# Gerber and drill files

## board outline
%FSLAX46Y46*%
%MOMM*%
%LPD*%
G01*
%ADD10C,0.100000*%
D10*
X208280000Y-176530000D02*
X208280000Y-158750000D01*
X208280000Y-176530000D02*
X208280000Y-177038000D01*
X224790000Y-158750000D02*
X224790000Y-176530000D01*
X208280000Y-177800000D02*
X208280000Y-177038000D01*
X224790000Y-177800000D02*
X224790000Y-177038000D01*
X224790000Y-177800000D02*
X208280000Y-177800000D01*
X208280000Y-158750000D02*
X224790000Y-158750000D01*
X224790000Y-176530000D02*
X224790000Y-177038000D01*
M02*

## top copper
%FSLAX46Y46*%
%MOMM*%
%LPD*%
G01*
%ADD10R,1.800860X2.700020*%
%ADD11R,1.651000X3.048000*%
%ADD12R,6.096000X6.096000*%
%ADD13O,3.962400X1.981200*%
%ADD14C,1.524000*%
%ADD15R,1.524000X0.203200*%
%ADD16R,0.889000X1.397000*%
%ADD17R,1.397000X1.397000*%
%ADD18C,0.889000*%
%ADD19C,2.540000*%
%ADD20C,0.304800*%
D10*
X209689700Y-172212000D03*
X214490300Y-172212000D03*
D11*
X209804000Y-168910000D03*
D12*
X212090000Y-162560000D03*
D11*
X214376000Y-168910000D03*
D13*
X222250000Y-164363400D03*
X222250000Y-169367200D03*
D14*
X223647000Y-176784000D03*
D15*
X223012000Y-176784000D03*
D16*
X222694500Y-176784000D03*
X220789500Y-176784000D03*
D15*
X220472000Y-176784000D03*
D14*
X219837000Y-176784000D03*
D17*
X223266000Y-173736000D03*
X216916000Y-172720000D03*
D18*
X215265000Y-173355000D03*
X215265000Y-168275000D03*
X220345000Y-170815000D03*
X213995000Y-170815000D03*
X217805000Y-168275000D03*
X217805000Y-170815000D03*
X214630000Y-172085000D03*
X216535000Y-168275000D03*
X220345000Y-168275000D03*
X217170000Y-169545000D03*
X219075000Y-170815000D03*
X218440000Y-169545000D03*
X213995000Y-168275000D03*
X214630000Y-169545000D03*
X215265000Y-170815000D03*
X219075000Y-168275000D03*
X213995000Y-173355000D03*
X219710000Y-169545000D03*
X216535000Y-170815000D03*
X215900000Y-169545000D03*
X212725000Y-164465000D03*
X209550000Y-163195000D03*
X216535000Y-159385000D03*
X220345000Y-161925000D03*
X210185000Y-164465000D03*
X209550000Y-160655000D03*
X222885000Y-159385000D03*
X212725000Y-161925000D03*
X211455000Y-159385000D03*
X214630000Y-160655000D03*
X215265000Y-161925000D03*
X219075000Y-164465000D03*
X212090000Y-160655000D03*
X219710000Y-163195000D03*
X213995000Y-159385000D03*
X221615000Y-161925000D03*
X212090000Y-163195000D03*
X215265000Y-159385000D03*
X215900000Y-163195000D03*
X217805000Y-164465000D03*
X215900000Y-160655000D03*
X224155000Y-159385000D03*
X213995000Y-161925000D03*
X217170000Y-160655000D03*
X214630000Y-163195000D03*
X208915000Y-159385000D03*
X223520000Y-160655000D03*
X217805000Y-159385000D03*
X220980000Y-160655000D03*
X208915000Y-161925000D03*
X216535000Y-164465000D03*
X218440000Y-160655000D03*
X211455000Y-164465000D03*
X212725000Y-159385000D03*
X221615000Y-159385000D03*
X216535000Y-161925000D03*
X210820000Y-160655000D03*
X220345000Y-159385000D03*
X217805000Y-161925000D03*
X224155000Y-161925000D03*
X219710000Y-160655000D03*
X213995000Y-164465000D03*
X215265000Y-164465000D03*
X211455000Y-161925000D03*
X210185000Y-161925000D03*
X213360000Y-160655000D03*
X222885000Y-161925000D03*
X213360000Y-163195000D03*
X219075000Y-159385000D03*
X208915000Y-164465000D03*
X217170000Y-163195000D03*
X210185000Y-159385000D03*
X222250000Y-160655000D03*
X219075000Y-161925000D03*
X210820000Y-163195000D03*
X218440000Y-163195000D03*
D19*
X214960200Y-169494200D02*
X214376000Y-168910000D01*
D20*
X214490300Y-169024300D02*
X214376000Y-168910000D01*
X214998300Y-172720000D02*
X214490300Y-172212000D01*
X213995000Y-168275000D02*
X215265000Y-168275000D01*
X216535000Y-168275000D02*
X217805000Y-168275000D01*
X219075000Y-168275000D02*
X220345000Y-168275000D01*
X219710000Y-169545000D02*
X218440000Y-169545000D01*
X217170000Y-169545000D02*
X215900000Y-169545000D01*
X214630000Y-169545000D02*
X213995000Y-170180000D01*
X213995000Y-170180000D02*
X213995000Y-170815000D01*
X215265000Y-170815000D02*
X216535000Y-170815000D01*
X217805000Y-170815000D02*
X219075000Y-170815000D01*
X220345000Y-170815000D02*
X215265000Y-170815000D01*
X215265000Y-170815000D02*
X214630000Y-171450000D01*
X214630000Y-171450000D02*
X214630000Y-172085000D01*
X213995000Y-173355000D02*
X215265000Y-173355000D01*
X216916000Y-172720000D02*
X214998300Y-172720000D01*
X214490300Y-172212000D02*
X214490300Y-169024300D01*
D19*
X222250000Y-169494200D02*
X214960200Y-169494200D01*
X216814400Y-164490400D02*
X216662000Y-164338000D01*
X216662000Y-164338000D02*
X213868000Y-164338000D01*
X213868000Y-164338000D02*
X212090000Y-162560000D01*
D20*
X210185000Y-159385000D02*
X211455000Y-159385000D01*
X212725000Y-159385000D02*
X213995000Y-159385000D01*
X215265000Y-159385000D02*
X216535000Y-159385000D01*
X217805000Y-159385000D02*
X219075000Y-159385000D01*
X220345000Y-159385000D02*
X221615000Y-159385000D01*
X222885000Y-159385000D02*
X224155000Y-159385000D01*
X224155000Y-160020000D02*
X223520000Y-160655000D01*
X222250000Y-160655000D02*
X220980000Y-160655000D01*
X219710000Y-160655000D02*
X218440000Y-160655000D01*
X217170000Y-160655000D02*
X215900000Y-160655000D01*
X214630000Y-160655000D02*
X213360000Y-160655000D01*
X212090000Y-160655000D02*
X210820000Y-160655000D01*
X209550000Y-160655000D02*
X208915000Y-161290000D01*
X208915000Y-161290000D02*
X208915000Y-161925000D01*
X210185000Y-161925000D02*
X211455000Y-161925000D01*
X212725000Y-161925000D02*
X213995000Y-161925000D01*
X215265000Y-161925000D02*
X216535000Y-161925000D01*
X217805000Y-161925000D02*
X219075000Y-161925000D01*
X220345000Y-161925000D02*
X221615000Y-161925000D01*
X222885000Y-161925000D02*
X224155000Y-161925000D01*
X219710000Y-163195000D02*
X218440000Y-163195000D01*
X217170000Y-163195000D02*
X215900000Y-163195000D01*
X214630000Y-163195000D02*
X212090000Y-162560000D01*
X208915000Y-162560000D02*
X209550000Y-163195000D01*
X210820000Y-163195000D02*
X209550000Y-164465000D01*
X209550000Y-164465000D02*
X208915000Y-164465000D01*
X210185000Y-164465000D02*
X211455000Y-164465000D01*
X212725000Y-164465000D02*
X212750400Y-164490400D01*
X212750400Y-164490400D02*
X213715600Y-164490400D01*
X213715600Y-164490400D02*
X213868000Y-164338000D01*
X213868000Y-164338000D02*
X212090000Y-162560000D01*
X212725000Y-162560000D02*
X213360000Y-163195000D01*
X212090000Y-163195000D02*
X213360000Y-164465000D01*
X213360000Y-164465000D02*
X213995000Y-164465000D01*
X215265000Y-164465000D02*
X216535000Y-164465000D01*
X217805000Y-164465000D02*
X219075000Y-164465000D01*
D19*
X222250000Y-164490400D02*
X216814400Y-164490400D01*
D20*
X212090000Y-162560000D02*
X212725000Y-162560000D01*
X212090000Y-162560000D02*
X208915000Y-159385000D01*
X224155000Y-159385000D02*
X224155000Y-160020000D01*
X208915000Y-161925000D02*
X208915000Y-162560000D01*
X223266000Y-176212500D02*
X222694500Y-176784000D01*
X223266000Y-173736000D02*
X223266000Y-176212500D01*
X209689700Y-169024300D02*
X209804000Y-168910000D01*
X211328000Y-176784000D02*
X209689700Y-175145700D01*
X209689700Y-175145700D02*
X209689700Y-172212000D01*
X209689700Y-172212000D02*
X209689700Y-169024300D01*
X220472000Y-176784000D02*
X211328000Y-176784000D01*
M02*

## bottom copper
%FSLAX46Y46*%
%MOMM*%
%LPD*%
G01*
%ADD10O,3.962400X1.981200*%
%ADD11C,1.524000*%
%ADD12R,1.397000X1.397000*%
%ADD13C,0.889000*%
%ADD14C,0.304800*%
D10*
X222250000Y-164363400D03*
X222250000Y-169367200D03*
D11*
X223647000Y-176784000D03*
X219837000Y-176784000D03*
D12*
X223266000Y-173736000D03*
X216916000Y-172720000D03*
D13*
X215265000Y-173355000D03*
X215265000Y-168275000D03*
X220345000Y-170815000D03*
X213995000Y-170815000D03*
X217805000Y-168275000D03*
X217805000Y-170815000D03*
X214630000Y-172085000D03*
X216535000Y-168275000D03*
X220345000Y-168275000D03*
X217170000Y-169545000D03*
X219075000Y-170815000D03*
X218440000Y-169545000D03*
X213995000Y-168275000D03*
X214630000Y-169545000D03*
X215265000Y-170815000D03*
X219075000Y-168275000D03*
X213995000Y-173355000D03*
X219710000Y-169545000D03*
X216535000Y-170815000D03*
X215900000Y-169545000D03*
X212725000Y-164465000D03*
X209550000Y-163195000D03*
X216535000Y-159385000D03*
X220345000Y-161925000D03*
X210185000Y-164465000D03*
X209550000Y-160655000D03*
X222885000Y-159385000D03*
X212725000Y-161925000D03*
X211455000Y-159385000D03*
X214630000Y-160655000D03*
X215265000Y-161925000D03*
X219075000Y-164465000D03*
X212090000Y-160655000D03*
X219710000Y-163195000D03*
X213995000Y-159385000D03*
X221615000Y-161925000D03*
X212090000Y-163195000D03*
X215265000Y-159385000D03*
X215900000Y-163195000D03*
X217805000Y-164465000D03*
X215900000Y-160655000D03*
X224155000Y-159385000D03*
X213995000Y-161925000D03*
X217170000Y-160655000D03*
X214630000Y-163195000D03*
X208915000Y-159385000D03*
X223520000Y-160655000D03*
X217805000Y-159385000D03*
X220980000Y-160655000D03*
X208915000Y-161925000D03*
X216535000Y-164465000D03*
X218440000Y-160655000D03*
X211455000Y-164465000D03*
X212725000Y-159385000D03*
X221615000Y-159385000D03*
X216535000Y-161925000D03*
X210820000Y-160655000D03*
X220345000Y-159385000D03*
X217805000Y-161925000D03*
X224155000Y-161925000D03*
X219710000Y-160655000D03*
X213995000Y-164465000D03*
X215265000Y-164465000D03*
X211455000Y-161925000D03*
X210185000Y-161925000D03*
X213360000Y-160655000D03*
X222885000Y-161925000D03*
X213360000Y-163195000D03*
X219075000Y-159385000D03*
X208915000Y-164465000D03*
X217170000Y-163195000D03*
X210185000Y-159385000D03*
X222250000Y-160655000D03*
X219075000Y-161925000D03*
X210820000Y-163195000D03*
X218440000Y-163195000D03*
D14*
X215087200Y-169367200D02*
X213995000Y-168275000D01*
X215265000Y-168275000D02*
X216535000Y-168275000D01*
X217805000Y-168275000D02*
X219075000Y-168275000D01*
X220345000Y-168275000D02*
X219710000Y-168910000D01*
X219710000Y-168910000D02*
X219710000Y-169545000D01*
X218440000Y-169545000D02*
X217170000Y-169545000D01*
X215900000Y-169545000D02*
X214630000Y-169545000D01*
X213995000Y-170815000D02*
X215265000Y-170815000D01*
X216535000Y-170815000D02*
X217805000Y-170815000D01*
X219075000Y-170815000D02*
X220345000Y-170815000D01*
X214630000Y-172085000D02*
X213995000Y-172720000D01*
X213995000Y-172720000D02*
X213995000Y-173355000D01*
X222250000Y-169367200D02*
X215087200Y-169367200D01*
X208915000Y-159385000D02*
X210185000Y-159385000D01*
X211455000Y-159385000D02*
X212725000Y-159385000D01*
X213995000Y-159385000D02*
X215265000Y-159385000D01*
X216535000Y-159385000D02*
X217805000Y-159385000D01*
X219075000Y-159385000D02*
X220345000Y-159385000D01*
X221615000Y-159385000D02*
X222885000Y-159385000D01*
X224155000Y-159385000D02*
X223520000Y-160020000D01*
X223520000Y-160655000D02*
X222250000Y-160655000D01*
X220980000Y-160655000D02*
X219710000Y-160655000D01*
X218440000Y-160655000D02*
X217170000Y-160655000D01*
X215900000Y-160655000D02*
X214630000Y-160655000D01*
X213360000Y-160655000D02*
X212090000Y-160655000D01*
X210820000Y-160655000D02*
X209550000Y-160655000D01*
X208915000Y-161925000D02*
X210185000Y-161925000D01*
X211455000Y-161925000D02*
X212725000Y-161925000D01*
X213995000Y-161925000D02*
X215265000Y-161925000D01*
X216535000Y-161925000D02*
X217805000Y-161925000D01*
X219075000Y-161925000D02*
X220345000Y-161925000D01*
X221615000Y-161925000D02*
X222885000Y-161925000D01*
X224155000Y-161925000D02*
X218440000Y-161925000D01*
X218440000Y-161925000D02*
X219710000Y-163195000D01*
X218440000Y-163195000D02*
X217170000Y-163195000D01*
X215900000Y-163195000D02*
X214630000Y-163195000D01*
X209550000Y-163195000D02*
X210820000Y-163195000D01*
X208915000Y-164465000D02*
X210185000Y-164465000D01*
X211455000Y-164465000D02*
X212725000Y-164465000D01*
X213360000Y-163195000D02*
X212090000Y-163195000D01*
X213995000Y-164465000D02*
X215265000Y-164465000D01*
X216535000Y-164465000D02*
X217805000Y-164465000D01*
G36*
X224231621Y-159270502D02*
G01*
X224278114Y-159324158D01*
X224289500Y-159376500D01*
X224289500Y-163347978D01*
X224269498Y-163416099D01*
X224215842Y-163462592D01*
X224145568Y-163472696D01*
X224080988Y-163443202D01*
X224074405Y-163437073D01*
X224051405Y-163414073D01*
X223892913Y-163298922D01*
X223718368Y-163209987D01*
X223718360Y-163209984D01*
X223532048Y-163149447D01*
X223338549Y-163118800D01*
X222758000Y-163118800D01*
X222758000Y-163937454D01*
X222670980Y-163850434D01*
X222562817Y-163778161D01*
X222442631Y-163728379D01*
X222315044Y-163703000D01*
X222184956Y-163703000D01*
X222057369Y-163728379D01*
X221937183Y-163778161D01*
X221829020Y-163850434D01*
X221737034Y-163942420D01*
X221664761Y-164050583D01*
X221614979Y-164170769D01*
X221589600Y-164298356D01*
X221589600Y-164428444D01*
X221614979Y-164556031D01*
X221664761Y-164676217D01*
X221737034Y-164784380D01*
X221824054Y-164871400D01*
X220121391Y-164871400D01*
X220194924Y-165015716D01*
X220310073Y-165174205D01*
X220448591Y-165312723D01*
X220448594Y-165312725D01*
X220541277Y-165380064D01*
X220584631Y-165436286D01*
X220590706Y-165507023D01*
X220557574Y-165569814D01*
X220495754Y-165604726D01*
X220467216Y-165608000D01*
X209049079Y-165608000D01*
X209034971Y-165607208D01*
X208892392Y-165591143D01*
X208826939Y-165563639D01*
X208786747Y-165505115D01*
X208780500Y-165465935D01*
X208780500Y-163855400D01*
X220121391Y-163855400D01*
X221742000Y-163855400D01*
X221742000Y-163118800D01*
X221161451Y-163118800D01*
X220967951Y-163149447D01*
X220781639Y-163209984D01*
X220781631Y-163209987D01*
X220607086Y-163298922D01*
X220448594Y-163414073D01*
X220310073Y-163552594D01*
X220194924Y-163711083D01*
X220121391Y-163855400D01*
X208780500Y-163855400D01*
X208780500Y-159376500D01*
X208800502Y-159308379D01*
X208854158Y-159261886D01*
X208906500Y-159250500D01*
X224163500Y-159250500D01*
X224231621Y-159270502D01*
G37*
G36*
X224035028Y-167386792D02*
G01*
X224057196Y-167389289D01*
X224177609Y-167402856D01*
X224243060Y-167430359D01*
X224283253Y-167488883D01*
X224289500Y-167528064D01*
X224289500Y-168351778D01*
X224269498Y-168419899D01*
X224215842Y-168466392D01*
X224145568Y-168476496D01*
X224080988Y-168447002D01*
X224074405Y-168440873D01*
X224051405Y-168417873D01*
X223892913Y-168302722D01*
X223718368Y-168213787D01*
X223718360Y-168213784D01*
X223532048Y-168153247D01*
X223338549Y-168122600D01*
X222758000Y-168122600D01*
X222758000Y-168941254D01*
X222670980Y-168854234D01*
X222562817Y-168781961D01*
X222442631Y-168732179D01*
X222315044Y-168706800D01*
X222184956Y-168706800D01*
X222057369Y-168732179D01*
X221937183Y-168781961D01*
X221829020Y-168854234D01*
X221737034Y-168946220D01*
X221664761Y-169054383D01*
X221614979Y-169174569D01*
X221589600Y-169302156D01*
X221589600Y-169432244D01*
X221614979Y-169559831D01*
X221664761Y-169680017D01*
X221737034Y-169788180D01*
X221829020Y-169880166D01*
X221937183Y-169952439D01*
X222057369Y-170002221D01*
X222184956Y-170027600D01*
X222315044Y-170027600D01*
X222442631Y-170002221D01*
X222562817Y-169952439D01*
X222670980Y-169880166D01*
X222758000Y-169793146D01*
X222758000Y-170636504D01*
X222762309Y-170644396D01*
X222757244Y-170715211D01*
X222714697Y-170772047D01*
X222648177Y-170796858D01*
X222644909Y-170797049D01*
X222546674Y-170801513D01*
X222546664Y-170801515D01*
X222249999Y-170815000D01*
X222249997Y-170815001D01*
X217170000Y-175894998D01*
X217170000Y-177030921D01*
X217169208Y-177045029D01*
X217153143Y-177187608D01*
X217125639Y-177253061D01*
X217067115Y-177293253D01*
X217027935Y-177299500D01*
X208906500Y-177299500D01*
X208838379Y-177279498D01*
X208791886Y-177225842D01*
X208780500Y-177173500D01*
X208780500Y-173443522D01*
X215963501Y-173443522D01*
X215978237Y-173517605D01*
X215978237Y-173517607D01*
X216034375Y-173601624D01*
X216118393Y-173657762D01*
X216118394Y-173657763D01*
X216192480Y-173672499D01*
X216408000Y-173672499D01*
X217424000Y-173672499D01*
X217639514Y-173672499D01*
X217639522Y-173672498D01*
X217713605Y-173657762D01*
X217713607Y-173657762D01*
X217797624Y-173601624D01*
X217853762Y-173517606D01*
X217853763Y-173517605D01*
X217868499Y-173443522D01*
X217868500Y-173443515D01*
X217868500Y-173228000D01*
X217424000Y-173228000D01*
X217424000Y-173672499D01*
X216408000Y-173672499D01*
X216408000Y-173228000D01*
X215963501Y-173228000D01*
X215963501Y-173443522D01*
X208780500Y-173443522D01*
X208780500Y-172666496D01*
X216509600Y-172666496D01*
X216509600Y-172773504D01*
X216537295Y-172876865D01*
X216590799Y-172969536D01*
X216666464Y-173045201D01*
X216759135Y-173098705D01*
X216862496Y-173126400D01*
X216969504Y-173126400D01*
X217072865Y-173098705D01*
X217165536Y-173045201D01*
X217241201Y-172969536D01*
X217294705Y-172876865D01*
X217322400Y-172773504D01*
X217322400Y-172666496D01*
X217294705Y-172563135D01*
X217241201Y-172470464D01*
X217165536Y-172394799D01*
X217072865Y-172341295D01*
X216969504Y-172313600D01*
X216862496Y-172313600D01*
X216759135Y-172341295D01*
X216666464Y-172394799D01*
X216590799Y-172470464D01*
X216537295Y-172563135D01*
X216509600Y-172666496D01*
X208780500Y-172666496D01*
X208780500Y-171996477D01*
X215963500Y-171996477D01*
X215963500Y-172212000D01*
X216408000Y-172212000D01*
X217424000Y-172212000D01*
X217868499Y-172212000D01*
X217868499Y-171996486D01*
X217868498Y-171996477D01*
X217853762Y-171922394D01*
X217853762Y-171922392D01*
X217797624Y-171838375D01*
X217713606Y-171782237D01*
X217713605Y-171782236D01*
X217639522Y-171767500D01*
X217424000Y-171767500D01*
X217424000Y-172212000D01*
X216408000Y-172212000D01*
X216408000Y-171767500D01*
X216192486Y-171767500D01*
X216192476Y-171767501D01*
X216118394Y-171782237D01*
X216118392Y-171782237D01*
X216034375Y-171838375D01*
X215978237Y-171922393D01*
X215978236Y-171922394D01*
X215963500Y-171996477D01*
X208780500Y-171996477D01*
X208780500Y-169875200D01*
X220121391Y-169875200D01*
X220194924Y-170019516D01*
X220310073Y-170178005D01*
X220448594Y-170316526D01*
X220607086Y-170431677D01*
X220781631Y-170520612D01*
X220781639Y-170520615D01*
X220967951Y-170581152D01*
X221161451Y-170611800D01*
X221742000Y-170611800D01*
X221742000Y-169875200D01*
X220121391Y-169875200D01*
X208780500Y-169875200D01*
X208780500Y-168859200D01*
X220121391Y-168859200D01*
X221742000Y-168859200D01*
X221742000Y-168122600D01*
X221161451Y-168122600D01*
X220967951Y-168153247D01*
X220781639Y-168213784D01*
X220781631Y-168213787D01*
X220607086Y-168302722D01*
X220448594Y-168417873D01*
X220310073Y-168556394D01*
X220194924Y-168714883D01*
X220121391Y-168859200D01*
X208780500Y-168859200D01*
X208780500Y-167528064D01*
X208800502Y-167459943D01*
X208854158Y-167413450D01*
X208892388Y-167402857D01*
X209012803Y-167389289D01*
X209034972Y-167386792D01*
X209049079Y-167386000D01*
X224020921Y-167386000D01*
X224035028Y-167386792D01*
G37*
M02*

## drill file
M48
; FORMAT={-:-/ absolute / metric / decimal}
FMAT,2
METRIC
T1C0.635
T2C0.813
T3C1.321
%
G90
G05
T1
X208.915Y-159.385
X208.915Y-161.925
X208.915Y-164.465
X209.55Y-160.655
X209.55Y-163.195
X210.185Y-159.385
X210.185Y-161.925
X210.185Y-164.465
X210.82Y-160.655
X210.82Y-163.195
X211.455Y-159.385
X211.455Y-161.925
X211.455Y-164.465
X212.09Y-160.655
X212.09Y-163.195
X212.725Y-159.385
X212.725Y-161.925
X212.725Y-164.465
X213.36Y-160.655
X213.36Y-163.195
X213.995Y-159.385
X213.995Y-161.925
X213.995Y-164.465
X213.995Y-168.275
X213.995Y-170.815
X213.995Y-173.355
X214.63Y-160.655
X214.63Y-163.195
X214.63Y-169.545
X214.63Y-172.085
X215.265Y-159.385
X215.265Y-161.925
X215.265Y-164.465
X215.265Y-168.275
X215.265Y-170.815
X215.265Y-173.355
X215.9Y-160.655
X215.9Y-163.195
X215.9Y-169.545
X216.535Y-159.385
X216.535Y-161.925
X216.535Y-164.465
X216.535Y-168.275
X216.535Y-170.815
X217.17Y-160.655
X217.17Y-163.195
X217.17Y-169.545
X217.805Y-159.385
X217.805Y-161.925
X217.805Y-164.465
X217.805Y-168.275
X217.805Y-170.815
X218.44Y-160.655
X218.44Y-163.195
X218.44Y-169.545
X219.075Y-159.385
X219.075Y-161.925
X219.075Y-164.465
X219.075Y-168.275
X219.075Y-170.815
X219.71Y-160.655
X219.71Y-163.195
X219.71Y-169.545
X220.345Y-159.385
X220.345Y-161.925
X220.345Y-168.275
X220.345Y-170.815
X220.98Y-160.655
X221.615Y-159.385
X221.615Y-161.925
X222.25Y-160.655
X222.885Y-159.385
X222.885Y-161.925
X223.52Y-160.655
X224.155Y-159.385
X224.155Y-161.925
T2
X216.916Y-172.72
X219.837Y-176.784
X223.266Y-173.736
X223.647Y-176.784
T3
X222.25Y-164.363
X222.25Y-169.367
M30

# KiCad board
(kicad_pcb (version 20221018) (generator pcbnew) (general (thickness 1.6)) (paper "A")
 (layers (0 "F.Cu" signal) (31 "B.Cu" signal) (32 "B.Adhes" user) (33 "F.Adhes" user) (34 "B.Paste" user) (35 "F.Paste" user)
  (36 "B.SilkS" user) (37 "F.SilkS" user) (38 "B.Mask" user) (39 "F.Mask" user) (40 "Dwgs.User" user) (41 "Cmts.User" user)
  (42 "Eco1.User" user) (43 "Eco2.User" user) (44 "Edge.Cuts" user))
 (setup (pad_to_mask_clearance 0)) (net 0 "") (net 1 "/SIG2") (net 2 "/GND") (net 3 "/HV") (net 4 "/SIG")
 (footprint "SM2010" (layer "F.Cu") (at 212.09 172.212)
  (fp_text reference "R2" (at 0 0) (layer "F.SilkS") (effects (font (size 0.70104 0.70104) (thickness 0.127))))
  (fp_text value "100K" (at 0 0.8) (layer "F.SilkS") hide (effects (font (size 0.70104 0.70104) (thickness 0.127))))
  (pad "1" smd rect (at -2.4003 0) (size 1.80086 2.70002) (layers "F.Cu" "F.Paste" "F.Mask") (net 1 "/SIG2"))
  (pad "2" smd rect (at 2.4003 0) (size 1.80086 2.70002) (layers "F.Cu" "F.Paste" "F.Mask") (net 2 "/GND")))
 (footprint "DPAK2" (layer "F.Cu") (at 212.09 168.91)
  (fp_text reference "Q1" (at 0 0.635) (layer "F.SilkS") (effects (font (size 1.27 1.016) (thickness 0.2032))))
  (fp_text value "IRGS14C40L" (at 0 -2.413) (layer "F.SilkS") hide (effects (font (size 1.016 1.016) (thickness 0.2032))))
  (pad "1" smd rect (at -2.286 0) (size 1.651 3.048) (layers "F.Cu" "F.Paste" "F.Mask") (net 1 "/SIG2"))
  (pad "2" smd rect (at 0 -6.35) (size 6.096 6.096) (layers "F.Cu" "F.Paste" "F.Mask") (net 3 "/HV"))
  (pad "3" smd rect (at 2.286 0) (size 1.651 3.048) (layers "F.Cu" "F.Paste" "F.Mask") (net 2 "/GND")))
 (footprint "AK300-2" (layer "F.Cu") (at 222.25 166.878 -90)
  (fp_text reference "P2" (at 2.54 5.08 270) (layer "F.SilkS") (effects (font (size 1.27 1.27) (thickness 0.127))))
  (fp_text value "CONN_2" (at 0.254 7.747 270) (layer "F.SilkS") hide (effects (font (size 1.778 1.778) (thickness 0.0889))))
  (pad "1" thru_hole oval (at -2.5146 0 270) (size 1.9812 3.9624) (drill 1.3208) (layers "*.Cu" "F.Paste" "F.SilkS" "F.Mask") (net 3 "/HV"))
  (pad "2" thru_hole oval (at 2.4892 0 270) (size 1.9812 3.9624) (drill 1.3208) (layers "*.Cu" "F.Paste" "F.SilkS" "F.Mask") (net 2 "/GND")))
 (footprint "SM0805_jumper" (layer "F.Cu") (at 221.742 176.784 180)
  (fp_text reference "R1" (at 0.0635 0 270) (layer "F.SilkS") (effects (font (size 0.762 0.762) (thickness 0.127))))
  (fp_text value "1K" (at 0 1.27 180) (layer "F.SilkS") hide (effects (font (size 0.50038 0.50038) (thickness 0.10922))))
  (pad "1" thru_hole circle (at -1.905 0 180) (size 1.524 1.524) (drill 0.8128) (layers "*.Cu" "*.Mask" "F.SilkS") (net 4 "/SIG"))
  (pad "1" smd rect (at -1.27 0 180) (size 1.524 0.2032) (layers "F.Cu" "F.Paste" "F.Mask") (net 4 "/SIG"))
  (pad "1" smd rect (at -0.9525 0 180) (size 0.889 1.397) (layers "F.Cu" "F.Paste" "F.Mask") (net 4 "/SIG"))
  (pad "2" smd rect (at 0.9525 0 180) (size 0.889 1.397) (layers "F.Cu" "F.Paste" "F.Mask") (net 1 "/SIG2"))
  (pad "2" smd rect (at 1.27 0 180) (size 1.524 0.2032) (layers "F.Cu" "F.Paste" "F.Mask") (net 1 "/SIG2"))
  (pad "2" thru_hole circle (at 1.905 0 180) (size 1.524 1.524) (drill 0.8128) (layers "*.Cu" "*.Mask" "F.SilkS") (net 1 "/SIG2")))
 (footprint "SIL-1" (layer "F.Cu") (at 223.266 173.736 180)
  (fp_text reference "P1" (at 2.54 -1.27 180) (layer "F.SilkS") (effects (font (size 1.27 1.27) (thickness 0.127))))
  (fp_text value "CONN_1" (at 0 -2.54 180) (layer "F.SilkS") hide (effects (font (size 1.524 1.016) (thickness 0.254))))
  (pad "1" thru_hole rect (at 0 0 180) (size 1.397 1.397) (drill 0.8128) (layers "*.Cu" "*.Mask" "F.SilkS") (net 4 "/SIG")))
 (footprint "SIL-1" (layer "F.Cu") (at 216.916 172.72)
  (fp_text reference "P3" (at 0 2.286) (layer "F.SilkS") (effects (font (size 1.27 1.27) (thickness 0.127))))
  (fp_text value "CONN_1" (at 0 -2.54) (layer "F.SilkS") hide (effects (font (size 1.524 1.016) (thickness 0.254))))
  (pad "1" thru_hole rect (at 0 0) (size 1.397 1.397) (drill 0.8128) (layers "*.Cu" "*.Mask" "F.SilkS") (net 2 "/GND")))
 (gr_line (start 208.28 176.53) (end 208.28 158.75) (stroke (width 0.1) (type solid)) (layer "Edge.Cuts"))
 (gr_line (start 208.28 176.53) (end 208.28 177.038) (stroke (width 0.1) (type solid)) (layer "Edge.Cuts"))
 (gr_line (start 224.79 158.75) (end 224.79 176.53) (stroke (width 0.1) (type solid)) (layer "Edge.Cuts"))
 (gr_line (start 208.28 177.8) (end 208.28 177.038) (stroke (width 0.1) (type solid)) (layer "Edge.Cuts"))
 (gr_line (start 224.79 177.8) (end 224.79 177.038) (stroke (width 0.1) (type solid)) (layer "Edge.Cuts"))
 (gr_line (start 224.79 177.8) (end 208.28 177.8) (stroke (width 0.1) (type solid)) (layer "Edge.Cuts"))
 (gr_line (start 208.28 158.75) (end 224.79 158.75) (stroke (width 0.1) (type solid)) (layer "Edge.Cuts"))
 (gr_line (start 224.79 176.53) (end 224.79 177.038) (stroke (width 0.1) (type solid)) (layer "Edge.Cuts"))
 (segment (start 214.9602 169.4942) (end 214.376 168.91) (width 2.54) (layer "F.Cu") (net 2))
 (segment (start 214.4903 169.0243) (end 214.376 168.91) (width 0.3048) (layer "F.Cu") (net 2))
 (segment (start 214.9983 172.72) (end 214.4903 172.212) (width 0.3048) (layer "F.Cu") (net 2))
 (segment (start 213.995 168.275) (end 215.265 168.275) (width 0.3048) (layer "F.Cu") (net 2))
 (segment (start 216.535 168.275) (end 217.805 168.275) (width 0.3048) (layer "F.Cu") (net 2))
 (segment (start 219.075 168.275) (end 220.345 168.275) (width 0.3048) (layer "F.Cu") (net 2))
 (segment (start 219.71 169.545) (end 218.44 169.545) (width 0.3048) (layer "F.Cu") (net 2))
 (segment (start 217.17 169.545) (end 215.9 169.545) (width 0.3048) (layer "F.Cu") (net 2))
 (segment (start 214.63 169.545) (end 213.995 170.18) (width 0.3048) (layer "F.Cu") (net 2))
 (segment (start 213.995 170.18) (end 213.995 170.815) (width 0.3048) (layer "F.Cu") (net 2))
 (segment (start 215.265 170.815) (end 216.535 170.815) (width 0.3048) (layer "F.Cu") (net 2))
 (segment (start 217.805 170.815) (end 219.075 170.815) (width 0.3048) (layer "F.Cu") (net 2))
 (segment (start 220.345 170.815) (end 215.265 170.815) (width 0.3048) (layer "F.Cu") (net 2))
 (segment (start 215.265 170.815) (end 214.63 171.45) (width 0.3048) (layer "F.Cu") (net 2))
 (segment (start 214.63 171.45) (end 214.63 172.085) (width 0.3048) (layer "F.Cu") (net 2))
 (segment (start 213.995 173.355) (end 215.265 173.355) (width 0.3048) (layer "F.Cu") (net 2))
 (segment (start 216.916 172.72) (end 214.9983 172.72) (width 0.3048) (layer "F.Cu") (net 2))
 (segment (start 214.4903 172.212) (end 214.4903 169.0243) (width 0.3048) (layer "F.Cu") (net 2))
 (segment (start 222.25 169.4942) (end 214.9602 169.4942) (width 2.54) (layer "F.Cu") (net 2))
 (via (at 215.265 173.355) (size 0.889) (drill 0.635) (layers "F.Cu" "B.Cu") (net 2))
 (via (at 215.265 168.275) (size 0.889) (drill 0.635) (layers "F.Cu" "B.Cu") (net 2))
 (via (at 220.345 170.815) (size 0.889) (drill 0.635) (layers "F.Cu" "B.Cu") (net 2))
 (via (at 213.995 170.815) (size 0.889) (drill 0.635) (layers "F.Cu" "B.Cu") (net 2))
 (via (at 217.805 168.275) (size 0.889) (drill 0.635) (layers "F.Cu" "B.Cu") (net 2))
 (via (at 217.805 170.815) (size 0.889) (drill 0.635) (layers "F.Cu" "B.Cu") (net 2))
 (via (at 214.63 172.085) (size 0.889) (drill 0.635) (layers "F.Cu" "B.Cu") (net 2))
 (via (at 216.535 168.275) (size 0.889) (drill 0.635) (layers "F.Cu" "B.Cu") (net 2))
 (via (at 220.345 168.275) (size 0.889) (drill 0.635) (layers "F.Cu" "B.Cu") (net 2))
 (via (at 217.17 169.545) (size 0.889) (drill 0.635) (layers "F.Cu" "B.Cu") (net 2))
 (via (at 219.075 170.815) (size 0.889) (drill 0.635) (layers "F.Cu" "B.Cu") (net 2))
 (via (at 218.44 169.545) (size 0.889) (drill 0.635) (layers "F.Cu" "B.Cu") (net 2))
 (via (at 213.995 168.275) (size 0.889) (drill 0.635) (layers "F.Cu" "B.Cu") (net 2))
 (via (at 214.63 169.545) (size 0.889) (drill 0.635) (layers "F.Cu" "B.Cu") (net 2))
 (via (at 215.265 170.815) (size 0.889) (drill 0.635) (layers "F.Cu" "B.Cu") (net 2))
 (via (at 219.075 168.275) (size 0.889) (drill 0.635) (layers "F.Cu" "B.Cu") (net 2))
 (via (at 213.995 173.355) (size 0.889) (drill 0.635) (layers "F.Cu" "B.Cu") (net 2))
 (via (at 219.71 169.545) (size 0.889) (drill 0.635) (layers "F.Cu" "B.Cu") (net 2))
 (via (at 216.535 170.815) (size 0.889) (drill 0.635) (layers "F.Cu" "B.Cu") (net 2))
 (via (at 215.9 169.545) (size 0.889) (drill 0.635) (layers "F.Cu" "B.Cu") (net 2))
 (segment (start 215.0872 169.3672) (end 213.995 168.275) (width 0.3048) (layer "B.Cu") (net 2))
 (segment (start 215.265 168.275) (end 216.535 168.275) (width 0.3048) (layer "B.Cu") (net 2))
 (segment (start 217.805 168.275) (end 219.075 168.275) (width 0.3048) (layer "B.Cu") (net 2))
 (segment (start 220.345 168.275) (end 219.71 168.91) (width 0.3048) (layer "B.Cu") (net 2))
 (segment (start 219.71 168.91) (end 219.71 169.545) (width 0.3048) (layer "B.Cu") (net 2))
 (segment (start 218.44 169.545) (end 217.17 169.545) (width 0.3048) (layer "B.Cu") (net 2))
 (segment (start 215.9 169.545) (end 214.63 169.545) (width 0.3048) (layer "B.Cu") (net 2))
 (segment (start 213.995 170.815) (end 215.265 170.815) (width 0.3048) (layer "B.Cu") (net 2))
 (segment (start 216.535 170.815) (end 217.805 170.815) (width 0.3048) (layer "B.Cu") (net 2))
 (segment (start 219.075 170.815) (end 220.345 170.815) (width 0.3048) (layer "B.Cu") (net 2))
 (segment (start 214.63 172.085) (end 213.995 172.72) (width 0.3048) (layer "B.Cu") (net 2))
 (segment (start 213.995 172.72) (end 213.995 173.355) (width 0.3048) (layer "B.Cu") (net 2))
 (segment (start 222.25 169.3672) (end 215.0872 169.3672) (width 0.3048) (layer "B.Cu") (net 2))
 (segment (start 216.8144 164.4904) (end 216.662 164.338) (width 2.54) (layer "F.Cu") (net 3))
 (segment (start 216.662 164.338) (end 213.868 164.338) (width 2.54) (layer "F.Cu") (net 3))
 (segment (start 213.868 164.338) (end 212.09 162.56) (width 2.54) (layer "F.Cu") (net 3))
 (segment (start 210.185 159.385) (end 211.455 159.385) (width 0.3048) (layer "F.Cu") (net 3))
 (segment (start 212.725 159.385) (end 213.995 159.385) (width 0.3048) (layer "F.Cu") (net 3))
 (segment (start 215.265 159.385) (end 216.535 159.385) (width 0.3048) (layer "F.Cu") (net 3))
 (segment (start 217.805 159.385) (end 219.075 159.385) (width 0.3048) (layer "F.Cu") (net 3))
 (segment (start 220.345 159.385) (end 221.615 159.385) (width 0.3048) (layer "F.Cu") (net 3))
 (segment (start 222.885 159.385) (end 224.155 159.385) (width 0.3048) (layer "F.Cu") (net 3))
 (segment (start 224.155 160.02) (end 223.52 160.655) (width 0.3048) (layer "F.Cu") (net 3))
 (segment (start 222.25 160.655) (end 220.98 160.655) (width 0.3048) (layer "F.Cu") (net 3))
 (segment (start 219.71 160.655) (end 218.44 160.655) (width 0.3048) (layer "F.Cu") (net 3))
 (segment (start 217.17 160.655) (end 215.9 160.655) (width 0.3048) (layer "F.Cu") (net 3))
 (segment (start 214.63 160.655) (end 213.36 160.655) (width 0.3048) (layer "F.Cu") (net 3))
 (segment (start 212.09 160.655) (end 210.82 160.655) (width 0.3048) (layer "F.Cu") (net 3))
 (segment (start 209.55 160.655) (end 208.915 161.29) (width 0.3048) (layer "F.Cu") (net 3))
 (segment (start 208.915 161.29) (end 208.915 161.925) (width 0.3048) (layer "F.Cu") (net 3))
 (segment (start 210.185 161.925) (end 211.455 161.925) (width 0.3048) (layer "F.Cu") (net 3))
 (segment (start 212.725 161.925) (end 213.995 161.925) (width 0.3048) (layer "F.Cu") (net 3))
 (segment (start 215.265 161.925) (end 216.535 161.925) (width 0.3048) (layer "F.Cu") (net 3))
 (segment (start 217.805 161.925) (end 219.075 161.925) (width 0.3048) (layer "F.Cu") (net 3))
 (segment (start 220.345 161.925) (end 221.615 161.925) (width 0.3048) (layer "F.Cu") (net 3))
 (segment (start 222.885 161.925) (end 224.155 161.925) (width 0.3048) (layer "F.Cu") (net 3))
 (segment (start 219.71 163.195) (end 218.44 163.195) (width 0.3048) (layer "F.Cu") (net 3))
 (segment (start 217.17 163.195) (end 215.9 163.195) (width 0.3048) (layer "F.Cu") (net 3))
 (segment (start 214.63 163.195) (end 212.09 162.56) (width 0.3048) (layer "F.Cu") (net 3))
 (segment (start 208.915 162.56) (end 209.55 163.195) (width 0.3048) (layer "F.Cu") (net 3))
 (segment (start 210.82 163.195) (end 209.55 164.465) (width 0.3048) (layer "F.Cu") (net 3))
 (segment (start 209.55 164.465) (end 208.915 164.465) (width 0.3048) (layer "F.Cu") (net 3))
 (segment (start 210.185 164.465) (end 211.455 164.465) (width 0.3048) (layer "F.Cu") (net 3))
 (segment (start 212.725 164.465) (end 212.7504 164.4904) (width 0.3048) (layer "F.Cu") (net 3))
 (segment (start 212.7504 164.4904) (end 213.7156 164.4904) (width 0.3048) (layer "F.Cu") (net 3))
 (segment (start 213.7156 164.4904) (end 213.868 164.338) (width 0.3048) (layer "F.Cu") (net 3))
 (segment (start 213.868 164.338) (end 212.09 162.56) (width 0.3048) (layer "F.Cu") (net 3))
 (segment (start 212.725 162.56) (end 213.36 163.195) (width 0.3048) (layer "F.Cu") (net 3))
 (segment (start 212.09 163.195) (end 213.36 164.465) (width 0.3048) (layer "F.Cu") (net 3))
 (segment (start 213.36 164.465) (end 213.995 164.465) (width 0.3048) (layer "F.Cu") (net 3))
 (segment (start 215.265 164.465) (end 216.535 164.465) (width 0.3048) (layer "F.Cu") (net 3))
 (segment (start 217.805 164.465) (end 219.075 164.465) (width 0.3048) (layer "F.Cu") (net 3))
 (segment (start 222.25 164.4904) (end 216.8144 164.4904) (width 2.54) (layer "F.Cu") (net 3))
 (segment (start 212.09 162.56) (end 212.725 162.56) (width 0.3048) (layer "F.Cu") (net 3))
 (segment (start 212.09 162.56) (end 208.915 159.385) (width 0.3048) (layer "F.Cu") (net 3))
 (segment (start 224.155 159.385) (end 224.155 160.02) (width 0.3048) (layer "F.Cu") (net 3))
 (segment (start 208.915 161.925) (end 208.915 162.56) (width 0.3048) (layer "F.Cu") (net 3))
 (via (at 212.725 164.465) (size 0.889) (drill 0.635) (layers "F.Cu" "B.Cu") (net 3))
 (via (at 209.55 163.195) (size 0.889) (drill 0.635) (layers "F.Cu" "B.Cu") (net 3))
 (via (at 216.535 159.385) (size 0.889) (drill 0.635) (layers "F.Cu" "B.Cu") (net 3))
 (via (at 220.345 161.925) (size 0.889) (drill 0.635) (layers "F.Cu" "B.Cu") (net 3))
 (via (at 210.185 164.465) (size 0.889) (drill 0.635) (layers "F.Cu" "B.Cu") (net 3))
 (via (at 209.55 160.655) (size 0.889) (drill 0.635) (layers "F.Cu" "B.Cu") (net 3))
 (via (at 222.885 159.385) (size 0.889) (drill 0.635) (layers "F.Cu" "B.Cu") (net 3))
 (via (at 212.725 161.925) (size 0.889) (drill 0.635) (layers "F.Cu" "B.Cu") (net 3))
 (via (at 211.455 159.385) (size 0.889) (drill 0.635) (layers "F.Cu" "B.Cu") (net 3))
 (via (at 214.63 160.655) (size 0.889) (drill 0.635) (layers "F.Cu" "B.Cu") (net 3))
 (via (at 215.265 161.925) (size 0.889) (drill 0.635) (layers "F.Cu" "B.Cu") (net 3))
 (via (at 219.075 164.465) (size 0.889) (drill 0.635) (layers "F.Cu" "B.Cu") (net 3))
 (via (at 212.09 160.655) (size 0.889) (drill 0.635) (layers "F.Cu" "B.Cu") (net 3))
 (via (at 219.71 163.195) (size 0.889) (drill 0.635) (layers "F.Cu" "B.Cu") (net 3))
 (via (at 213.995 159.385) (size 0.889) (drill 0.635) (layers "F.Cu" "B.Cu") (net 3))
 (via (at 221.615 161.925) (size 0.889) (drill 0.635) (layers "F.Cu" "B.Cu") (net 3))
 (via (at 212.09 163.195) (size 0.889) (drill 0.635) (layers "F.Cu" "B.Cu") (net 3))
 (via (at 215.265 159.385) (size 0.889) (drill 0.635) (layers "F.Cu" "B.Cu") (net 3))
 (via (at 215.9 163.195) (size 0.889) (drill 0.635) (layers "F.Cu" "B.Cu") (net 3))
 (via (at 217.805 164.465) (size 0.889) (drill 0.635) (layers "F.Cu" "B.Cu") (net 3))
 (via (at 215.9 160.655) (size 0.889) (drill 0.635) (layers "F.Cu" "B.Cu") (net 3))
 (via (at 224.155 159.385) (size 0.889) (drill 0.635) (layers "F.Cu" "B.Cu") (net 3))
 (via (at 213.995 161.925) (size 0.889) (drill 0.635) (layers "F.Cu" "B.Cu") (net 3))
 (via (at 217.17 160.655) (size 0.889) (drill 0.635) (layers "F.Cu" "B.Cu") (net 3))
 (via (at 214.63 163.195) (size 0.889) (drill 0.635) (layers "F.Cu" "B.Cu") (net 3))
 (via (at 208.915 159.385) (size 0.889) (drill 0.635) (layers "F.Cu" "B.Cu") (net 3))
 (via (at 223.52 160.655) (size 0.889) (drill 0.635) (layers "F.Cu" "B.Cu") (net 3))
 (via (at 217.805 159.385) (size 0.889) (drill 0.635) (layers "F.Cu" "B.Cu") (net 3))
 (via (at 220.98 160.655) (size 0.889) (drill 0.635) (layers "F.Cu" "B.Cu") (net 3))
 (via (at 208.915 161.925) (size 0.889) (drill 0.635) (layers "F.Cu" "B.Cu") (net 3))
 (via (at 216.535 164.465) (size 0.889) (drill 0.635) (layers "F.Cu" "B.Cu") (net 3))
 (via (at 218.44 160.655) (size 0.889) (drill 0.635) (layers "F.Cu" "B.Cu") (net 3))
 (via (at 211.455 164.465) (size 0.889) (drill 0.635) (layers "F.Cu" "B.Cu") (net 3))
 (via (at 212.725 159.385) (size 0.889) (drill 0.635) (layers "F.Cu" "B.Cu") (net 3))
 (via (at 221.615 159.385) (size 0.889) (drill 0.635) (layers "F.Cu" "B.Cu") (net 3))
 (via (at 216.535 161.925) (size 0.889) (drill 0.635) (layers "F.Cu" "B.Cu") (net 3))
 (via (at 210.82 160.655) (size 0.889) (drill 0.635) (layers "F.Cu" "B.Cu") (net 3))
 (via (at 220.345 159.385) (size 0.889) (drill 0.635) (layers "F.Cu" "B.Cu") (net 3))
 (via (at 217.805 161.925) (size 0.889) (drill 0.635) (layers "F.Cu" "B.Cu") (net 3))
 (via (at 224.155 161.925) (size 0.889) (drill 0.635) (layers "F.Cu" "B.Cu") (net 3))
 (via (at 219.71 160.655) (size 0.889) (drill 0.635) (layers "F.Cu" "B.Cu") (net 3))
 (via (at 213.995 164.465) (size 0.889) (drill 0.635) (layers "F.Cu" "B.Cu") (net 3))
 (via (at 215.265 164.465) (size 0.889) (drill 0.635) (layers "F.Cu" "B.Cu") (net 3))
 (via (at 211.455 161.925) (size 0.889) (drill 0.635) (layers "F.Cu" "B.Cu") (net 3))
 (via (at 210.185 161.925) (size 0.889) (drill 0.635) (layers "F.Cu" "B.Cu") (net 3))
 (via (at 213.36 160.655) (size 0.889) (drill 0.635) (layers "F.Cu" "B.Cu") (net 3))
 (via (at 222.885 161.925) (size 0.889) (drill 0.635) (layers "F.Cu" "B.Cu") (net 3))
 (via (at 213.36 163.195) (size 0.889) (drill 0.635) (layers "F.Cu" "B.Cu") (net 3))
 (via (at 219.075 159.385) (size 0.889) (drill 0.635) (layers "F.Cu" "B.Cu") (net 3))
 (via (at 208.915 164.465) (size 0.889) (drill 0.635) (layers "F.Cu" "B.Cu") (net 3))
 (via (at 217.17 163.195) (size 0.889) (drill 0.635) (layers "F.Cu" "B.Cu") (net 3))
 (via (at 210.185 159.385) (size 0.889) (drill 0.635) (layers "F.Cu" "B.Cu") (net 3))
 (via (at 222.25 160.655) (size 0.889) (drill 0.635) (layers "F.Cu" "B.Cu") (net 3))
 (via (at 219.075 161.925) (size 0.889) (drill 0.635) (layers "F.Cu" "B.Cu") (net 3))
 (via (at 210.82 163.195) (size 0.889) (drill 0.635) (layers "F.Cu" "B.Cu") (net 3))
 (via (at 218.44 163.195) (size 0.889) (drill 0.635) (layers "F.Cu" "B.Cu") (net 3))
 (segment (start 208.915 159.385) (end 210.185 159.385) (width 0.3048) (layer "B.Cu") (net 3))
 (segment (start 211.455 159.385) (end 212.725 159.385) (width 0.3048) (layer "B.Cu") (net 3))
 (segment (start 213.995 159.385) (end 215.265 159.385) (width 0.3048) (layer "B.Cu") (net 3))
 (segment (start 216.535 159.385) (end 217.805 159.385) (width 0.3048) (layer "B.Cu") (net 3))
 (segment (start 219.075 159.385) (end 220.345 159.385) (width 0.3048) (layer "B.Cu") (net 3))
 (segment (start 221.615 159.385) (end 222.885 159.385) (width 0.3048) (layer "B.Cu") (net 3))
 (segment (start 224.155 159.385) (end 223.52 160.02) (width 0.3048) (layer "B.Cu") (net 3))
 (segment (start 223.52 160.655) (end 222.25 160.655) (width 0.3048) (layer "B.Cu") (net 3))
 (segment (start 220.98 160.655) (end 219.71 160.655) (width 0.3048) (layer "B.Cu") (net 3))
 (segment (start 218.44 160.655) (end 217.17 160.655) (width 0.3048) (layer "B.Cu") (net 3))
 (segment (start 215.9 160.655) (end 214.63 160.655) (width 0.3048) (layer "B.Cu") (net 3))
 (segment (start 213.36 160.655) (end 212.09 160.655) (width 0.3048) (layer "B.Cu") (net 3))
 (segment (start 210.82 160.655) (end 209.55 160.655) (width 0.3048) (layer "B.Cu") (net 3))
 (segment (start 208.915 161.925) (end 210.185 161.925) (width 0.3048) (layer "B.Cu") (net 3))
 (segment (start 211.455 161.925) (end 212.725 161.925) (width 0.3048) (layer "B.Cu") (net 3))
 (segment (start 213.995 161.925) (end 215.265 161.925) (width 0.3048) (layer "B.Cu") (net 3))
 (segment (start 216.535 161.925) (end 217.805 161.925) (width 0.3048) (layer "B.Cu") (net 3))
 (segment (start 219.075 161.925) (end 220.345 161.925) (width 0.3048) (layer "B.Cu") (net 3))
 (segment (start 221.615 161.925) (end 222.885 161.925) (width 0.3048) (layer "B.Cu") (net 3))
 (segment (start 224.155 161.925) (end 218.44 161.925) (width 0.3048) (layer "B.Cu") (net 3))
 (segment (start 218.44 161.925) (end 219.71 163.195) (width 0.3048) (layer "B.Cu") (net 3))
 (segment (start 218.44 163.195) (end 217.17 163.195) (width 0.3048) (layer "B.Cu") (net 3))
 (segment (start 215.9 163.195) (end 214.63 163.195) (width 0.3048) (layer "B.Cu") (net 3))
 (segment (start 209.55 163.195) (end 210.82 163.195) (width 0.3048) (layer "B.Cu") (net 3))
 (segment (start 208.915 164.465) (end 210.185 164.465) (width 0.3048) (layer "B.Cu") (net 3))
 (segment (start 211.455 164.465) (end 212.725 164.465) (width 0.3048) (layer "B.Cu") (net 3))
 (segment (start 213.36 163.195) (end 212.09 163.195) (width 0.3048) (layer "B.Cu") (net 3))
 (segment (start 213.995 164.465) (end 215.265 164.465) (width 0.3048) (layer "B.Cu") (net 3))
 (segment (start 216.535 164.465) (end 217.805 164.465) (width 0.3048) (layer "B.Cu") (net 3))
 (segment (start 223.266 176.2125) (end 222.6945 176.784) (width 0.3048) (layer "F.Cu") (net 4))
 (segment (start 223.266 173.736) (end 223.266 176.2125) (width 0.3048) (layer "F.Cu") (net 4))
 (segment (start 209.6897 169.0243) (end 209.804 168.91) (width 0.3048) (layer "F.Cu") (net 1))
 (segment (start 211.328 176.784) (end 209.6897 175.1457) (width 0.3048) (layer "F.Cu") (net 1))
 (segment (start 209.6897 175.1457) (end 209.6897 172.212) (width 0.3048) (layer "F.Cu") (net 1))
 (segment (start 209.6897 172.212) (end 209.6897 169.0243) (width 0.3048) (layer "F.Cu") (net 1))
 (segment (start 220.472 176.784) (end 211.328 176.784) (width 0.3048) (layer "F.Cu") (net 1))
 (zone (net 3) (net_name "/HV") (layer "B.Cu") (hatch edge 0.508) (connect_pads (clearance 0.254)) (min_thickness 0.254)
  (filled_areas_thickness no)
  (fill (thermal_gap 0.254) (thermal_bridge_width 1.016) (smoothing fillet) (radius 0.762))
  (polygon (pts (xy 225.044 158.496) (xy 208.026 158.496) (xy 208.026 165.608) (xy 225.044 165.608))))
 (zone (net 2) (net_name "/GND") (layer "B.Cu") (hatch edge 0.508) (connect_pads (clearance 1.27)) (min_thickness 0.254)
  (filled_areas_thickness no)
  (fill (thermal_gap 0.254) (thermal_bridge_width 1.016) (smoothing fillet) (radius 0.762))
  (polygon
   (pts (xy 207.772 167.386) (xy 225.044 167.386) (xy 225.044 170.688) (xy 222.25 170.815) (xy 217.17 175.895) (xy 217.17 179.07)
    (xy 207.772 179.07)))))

